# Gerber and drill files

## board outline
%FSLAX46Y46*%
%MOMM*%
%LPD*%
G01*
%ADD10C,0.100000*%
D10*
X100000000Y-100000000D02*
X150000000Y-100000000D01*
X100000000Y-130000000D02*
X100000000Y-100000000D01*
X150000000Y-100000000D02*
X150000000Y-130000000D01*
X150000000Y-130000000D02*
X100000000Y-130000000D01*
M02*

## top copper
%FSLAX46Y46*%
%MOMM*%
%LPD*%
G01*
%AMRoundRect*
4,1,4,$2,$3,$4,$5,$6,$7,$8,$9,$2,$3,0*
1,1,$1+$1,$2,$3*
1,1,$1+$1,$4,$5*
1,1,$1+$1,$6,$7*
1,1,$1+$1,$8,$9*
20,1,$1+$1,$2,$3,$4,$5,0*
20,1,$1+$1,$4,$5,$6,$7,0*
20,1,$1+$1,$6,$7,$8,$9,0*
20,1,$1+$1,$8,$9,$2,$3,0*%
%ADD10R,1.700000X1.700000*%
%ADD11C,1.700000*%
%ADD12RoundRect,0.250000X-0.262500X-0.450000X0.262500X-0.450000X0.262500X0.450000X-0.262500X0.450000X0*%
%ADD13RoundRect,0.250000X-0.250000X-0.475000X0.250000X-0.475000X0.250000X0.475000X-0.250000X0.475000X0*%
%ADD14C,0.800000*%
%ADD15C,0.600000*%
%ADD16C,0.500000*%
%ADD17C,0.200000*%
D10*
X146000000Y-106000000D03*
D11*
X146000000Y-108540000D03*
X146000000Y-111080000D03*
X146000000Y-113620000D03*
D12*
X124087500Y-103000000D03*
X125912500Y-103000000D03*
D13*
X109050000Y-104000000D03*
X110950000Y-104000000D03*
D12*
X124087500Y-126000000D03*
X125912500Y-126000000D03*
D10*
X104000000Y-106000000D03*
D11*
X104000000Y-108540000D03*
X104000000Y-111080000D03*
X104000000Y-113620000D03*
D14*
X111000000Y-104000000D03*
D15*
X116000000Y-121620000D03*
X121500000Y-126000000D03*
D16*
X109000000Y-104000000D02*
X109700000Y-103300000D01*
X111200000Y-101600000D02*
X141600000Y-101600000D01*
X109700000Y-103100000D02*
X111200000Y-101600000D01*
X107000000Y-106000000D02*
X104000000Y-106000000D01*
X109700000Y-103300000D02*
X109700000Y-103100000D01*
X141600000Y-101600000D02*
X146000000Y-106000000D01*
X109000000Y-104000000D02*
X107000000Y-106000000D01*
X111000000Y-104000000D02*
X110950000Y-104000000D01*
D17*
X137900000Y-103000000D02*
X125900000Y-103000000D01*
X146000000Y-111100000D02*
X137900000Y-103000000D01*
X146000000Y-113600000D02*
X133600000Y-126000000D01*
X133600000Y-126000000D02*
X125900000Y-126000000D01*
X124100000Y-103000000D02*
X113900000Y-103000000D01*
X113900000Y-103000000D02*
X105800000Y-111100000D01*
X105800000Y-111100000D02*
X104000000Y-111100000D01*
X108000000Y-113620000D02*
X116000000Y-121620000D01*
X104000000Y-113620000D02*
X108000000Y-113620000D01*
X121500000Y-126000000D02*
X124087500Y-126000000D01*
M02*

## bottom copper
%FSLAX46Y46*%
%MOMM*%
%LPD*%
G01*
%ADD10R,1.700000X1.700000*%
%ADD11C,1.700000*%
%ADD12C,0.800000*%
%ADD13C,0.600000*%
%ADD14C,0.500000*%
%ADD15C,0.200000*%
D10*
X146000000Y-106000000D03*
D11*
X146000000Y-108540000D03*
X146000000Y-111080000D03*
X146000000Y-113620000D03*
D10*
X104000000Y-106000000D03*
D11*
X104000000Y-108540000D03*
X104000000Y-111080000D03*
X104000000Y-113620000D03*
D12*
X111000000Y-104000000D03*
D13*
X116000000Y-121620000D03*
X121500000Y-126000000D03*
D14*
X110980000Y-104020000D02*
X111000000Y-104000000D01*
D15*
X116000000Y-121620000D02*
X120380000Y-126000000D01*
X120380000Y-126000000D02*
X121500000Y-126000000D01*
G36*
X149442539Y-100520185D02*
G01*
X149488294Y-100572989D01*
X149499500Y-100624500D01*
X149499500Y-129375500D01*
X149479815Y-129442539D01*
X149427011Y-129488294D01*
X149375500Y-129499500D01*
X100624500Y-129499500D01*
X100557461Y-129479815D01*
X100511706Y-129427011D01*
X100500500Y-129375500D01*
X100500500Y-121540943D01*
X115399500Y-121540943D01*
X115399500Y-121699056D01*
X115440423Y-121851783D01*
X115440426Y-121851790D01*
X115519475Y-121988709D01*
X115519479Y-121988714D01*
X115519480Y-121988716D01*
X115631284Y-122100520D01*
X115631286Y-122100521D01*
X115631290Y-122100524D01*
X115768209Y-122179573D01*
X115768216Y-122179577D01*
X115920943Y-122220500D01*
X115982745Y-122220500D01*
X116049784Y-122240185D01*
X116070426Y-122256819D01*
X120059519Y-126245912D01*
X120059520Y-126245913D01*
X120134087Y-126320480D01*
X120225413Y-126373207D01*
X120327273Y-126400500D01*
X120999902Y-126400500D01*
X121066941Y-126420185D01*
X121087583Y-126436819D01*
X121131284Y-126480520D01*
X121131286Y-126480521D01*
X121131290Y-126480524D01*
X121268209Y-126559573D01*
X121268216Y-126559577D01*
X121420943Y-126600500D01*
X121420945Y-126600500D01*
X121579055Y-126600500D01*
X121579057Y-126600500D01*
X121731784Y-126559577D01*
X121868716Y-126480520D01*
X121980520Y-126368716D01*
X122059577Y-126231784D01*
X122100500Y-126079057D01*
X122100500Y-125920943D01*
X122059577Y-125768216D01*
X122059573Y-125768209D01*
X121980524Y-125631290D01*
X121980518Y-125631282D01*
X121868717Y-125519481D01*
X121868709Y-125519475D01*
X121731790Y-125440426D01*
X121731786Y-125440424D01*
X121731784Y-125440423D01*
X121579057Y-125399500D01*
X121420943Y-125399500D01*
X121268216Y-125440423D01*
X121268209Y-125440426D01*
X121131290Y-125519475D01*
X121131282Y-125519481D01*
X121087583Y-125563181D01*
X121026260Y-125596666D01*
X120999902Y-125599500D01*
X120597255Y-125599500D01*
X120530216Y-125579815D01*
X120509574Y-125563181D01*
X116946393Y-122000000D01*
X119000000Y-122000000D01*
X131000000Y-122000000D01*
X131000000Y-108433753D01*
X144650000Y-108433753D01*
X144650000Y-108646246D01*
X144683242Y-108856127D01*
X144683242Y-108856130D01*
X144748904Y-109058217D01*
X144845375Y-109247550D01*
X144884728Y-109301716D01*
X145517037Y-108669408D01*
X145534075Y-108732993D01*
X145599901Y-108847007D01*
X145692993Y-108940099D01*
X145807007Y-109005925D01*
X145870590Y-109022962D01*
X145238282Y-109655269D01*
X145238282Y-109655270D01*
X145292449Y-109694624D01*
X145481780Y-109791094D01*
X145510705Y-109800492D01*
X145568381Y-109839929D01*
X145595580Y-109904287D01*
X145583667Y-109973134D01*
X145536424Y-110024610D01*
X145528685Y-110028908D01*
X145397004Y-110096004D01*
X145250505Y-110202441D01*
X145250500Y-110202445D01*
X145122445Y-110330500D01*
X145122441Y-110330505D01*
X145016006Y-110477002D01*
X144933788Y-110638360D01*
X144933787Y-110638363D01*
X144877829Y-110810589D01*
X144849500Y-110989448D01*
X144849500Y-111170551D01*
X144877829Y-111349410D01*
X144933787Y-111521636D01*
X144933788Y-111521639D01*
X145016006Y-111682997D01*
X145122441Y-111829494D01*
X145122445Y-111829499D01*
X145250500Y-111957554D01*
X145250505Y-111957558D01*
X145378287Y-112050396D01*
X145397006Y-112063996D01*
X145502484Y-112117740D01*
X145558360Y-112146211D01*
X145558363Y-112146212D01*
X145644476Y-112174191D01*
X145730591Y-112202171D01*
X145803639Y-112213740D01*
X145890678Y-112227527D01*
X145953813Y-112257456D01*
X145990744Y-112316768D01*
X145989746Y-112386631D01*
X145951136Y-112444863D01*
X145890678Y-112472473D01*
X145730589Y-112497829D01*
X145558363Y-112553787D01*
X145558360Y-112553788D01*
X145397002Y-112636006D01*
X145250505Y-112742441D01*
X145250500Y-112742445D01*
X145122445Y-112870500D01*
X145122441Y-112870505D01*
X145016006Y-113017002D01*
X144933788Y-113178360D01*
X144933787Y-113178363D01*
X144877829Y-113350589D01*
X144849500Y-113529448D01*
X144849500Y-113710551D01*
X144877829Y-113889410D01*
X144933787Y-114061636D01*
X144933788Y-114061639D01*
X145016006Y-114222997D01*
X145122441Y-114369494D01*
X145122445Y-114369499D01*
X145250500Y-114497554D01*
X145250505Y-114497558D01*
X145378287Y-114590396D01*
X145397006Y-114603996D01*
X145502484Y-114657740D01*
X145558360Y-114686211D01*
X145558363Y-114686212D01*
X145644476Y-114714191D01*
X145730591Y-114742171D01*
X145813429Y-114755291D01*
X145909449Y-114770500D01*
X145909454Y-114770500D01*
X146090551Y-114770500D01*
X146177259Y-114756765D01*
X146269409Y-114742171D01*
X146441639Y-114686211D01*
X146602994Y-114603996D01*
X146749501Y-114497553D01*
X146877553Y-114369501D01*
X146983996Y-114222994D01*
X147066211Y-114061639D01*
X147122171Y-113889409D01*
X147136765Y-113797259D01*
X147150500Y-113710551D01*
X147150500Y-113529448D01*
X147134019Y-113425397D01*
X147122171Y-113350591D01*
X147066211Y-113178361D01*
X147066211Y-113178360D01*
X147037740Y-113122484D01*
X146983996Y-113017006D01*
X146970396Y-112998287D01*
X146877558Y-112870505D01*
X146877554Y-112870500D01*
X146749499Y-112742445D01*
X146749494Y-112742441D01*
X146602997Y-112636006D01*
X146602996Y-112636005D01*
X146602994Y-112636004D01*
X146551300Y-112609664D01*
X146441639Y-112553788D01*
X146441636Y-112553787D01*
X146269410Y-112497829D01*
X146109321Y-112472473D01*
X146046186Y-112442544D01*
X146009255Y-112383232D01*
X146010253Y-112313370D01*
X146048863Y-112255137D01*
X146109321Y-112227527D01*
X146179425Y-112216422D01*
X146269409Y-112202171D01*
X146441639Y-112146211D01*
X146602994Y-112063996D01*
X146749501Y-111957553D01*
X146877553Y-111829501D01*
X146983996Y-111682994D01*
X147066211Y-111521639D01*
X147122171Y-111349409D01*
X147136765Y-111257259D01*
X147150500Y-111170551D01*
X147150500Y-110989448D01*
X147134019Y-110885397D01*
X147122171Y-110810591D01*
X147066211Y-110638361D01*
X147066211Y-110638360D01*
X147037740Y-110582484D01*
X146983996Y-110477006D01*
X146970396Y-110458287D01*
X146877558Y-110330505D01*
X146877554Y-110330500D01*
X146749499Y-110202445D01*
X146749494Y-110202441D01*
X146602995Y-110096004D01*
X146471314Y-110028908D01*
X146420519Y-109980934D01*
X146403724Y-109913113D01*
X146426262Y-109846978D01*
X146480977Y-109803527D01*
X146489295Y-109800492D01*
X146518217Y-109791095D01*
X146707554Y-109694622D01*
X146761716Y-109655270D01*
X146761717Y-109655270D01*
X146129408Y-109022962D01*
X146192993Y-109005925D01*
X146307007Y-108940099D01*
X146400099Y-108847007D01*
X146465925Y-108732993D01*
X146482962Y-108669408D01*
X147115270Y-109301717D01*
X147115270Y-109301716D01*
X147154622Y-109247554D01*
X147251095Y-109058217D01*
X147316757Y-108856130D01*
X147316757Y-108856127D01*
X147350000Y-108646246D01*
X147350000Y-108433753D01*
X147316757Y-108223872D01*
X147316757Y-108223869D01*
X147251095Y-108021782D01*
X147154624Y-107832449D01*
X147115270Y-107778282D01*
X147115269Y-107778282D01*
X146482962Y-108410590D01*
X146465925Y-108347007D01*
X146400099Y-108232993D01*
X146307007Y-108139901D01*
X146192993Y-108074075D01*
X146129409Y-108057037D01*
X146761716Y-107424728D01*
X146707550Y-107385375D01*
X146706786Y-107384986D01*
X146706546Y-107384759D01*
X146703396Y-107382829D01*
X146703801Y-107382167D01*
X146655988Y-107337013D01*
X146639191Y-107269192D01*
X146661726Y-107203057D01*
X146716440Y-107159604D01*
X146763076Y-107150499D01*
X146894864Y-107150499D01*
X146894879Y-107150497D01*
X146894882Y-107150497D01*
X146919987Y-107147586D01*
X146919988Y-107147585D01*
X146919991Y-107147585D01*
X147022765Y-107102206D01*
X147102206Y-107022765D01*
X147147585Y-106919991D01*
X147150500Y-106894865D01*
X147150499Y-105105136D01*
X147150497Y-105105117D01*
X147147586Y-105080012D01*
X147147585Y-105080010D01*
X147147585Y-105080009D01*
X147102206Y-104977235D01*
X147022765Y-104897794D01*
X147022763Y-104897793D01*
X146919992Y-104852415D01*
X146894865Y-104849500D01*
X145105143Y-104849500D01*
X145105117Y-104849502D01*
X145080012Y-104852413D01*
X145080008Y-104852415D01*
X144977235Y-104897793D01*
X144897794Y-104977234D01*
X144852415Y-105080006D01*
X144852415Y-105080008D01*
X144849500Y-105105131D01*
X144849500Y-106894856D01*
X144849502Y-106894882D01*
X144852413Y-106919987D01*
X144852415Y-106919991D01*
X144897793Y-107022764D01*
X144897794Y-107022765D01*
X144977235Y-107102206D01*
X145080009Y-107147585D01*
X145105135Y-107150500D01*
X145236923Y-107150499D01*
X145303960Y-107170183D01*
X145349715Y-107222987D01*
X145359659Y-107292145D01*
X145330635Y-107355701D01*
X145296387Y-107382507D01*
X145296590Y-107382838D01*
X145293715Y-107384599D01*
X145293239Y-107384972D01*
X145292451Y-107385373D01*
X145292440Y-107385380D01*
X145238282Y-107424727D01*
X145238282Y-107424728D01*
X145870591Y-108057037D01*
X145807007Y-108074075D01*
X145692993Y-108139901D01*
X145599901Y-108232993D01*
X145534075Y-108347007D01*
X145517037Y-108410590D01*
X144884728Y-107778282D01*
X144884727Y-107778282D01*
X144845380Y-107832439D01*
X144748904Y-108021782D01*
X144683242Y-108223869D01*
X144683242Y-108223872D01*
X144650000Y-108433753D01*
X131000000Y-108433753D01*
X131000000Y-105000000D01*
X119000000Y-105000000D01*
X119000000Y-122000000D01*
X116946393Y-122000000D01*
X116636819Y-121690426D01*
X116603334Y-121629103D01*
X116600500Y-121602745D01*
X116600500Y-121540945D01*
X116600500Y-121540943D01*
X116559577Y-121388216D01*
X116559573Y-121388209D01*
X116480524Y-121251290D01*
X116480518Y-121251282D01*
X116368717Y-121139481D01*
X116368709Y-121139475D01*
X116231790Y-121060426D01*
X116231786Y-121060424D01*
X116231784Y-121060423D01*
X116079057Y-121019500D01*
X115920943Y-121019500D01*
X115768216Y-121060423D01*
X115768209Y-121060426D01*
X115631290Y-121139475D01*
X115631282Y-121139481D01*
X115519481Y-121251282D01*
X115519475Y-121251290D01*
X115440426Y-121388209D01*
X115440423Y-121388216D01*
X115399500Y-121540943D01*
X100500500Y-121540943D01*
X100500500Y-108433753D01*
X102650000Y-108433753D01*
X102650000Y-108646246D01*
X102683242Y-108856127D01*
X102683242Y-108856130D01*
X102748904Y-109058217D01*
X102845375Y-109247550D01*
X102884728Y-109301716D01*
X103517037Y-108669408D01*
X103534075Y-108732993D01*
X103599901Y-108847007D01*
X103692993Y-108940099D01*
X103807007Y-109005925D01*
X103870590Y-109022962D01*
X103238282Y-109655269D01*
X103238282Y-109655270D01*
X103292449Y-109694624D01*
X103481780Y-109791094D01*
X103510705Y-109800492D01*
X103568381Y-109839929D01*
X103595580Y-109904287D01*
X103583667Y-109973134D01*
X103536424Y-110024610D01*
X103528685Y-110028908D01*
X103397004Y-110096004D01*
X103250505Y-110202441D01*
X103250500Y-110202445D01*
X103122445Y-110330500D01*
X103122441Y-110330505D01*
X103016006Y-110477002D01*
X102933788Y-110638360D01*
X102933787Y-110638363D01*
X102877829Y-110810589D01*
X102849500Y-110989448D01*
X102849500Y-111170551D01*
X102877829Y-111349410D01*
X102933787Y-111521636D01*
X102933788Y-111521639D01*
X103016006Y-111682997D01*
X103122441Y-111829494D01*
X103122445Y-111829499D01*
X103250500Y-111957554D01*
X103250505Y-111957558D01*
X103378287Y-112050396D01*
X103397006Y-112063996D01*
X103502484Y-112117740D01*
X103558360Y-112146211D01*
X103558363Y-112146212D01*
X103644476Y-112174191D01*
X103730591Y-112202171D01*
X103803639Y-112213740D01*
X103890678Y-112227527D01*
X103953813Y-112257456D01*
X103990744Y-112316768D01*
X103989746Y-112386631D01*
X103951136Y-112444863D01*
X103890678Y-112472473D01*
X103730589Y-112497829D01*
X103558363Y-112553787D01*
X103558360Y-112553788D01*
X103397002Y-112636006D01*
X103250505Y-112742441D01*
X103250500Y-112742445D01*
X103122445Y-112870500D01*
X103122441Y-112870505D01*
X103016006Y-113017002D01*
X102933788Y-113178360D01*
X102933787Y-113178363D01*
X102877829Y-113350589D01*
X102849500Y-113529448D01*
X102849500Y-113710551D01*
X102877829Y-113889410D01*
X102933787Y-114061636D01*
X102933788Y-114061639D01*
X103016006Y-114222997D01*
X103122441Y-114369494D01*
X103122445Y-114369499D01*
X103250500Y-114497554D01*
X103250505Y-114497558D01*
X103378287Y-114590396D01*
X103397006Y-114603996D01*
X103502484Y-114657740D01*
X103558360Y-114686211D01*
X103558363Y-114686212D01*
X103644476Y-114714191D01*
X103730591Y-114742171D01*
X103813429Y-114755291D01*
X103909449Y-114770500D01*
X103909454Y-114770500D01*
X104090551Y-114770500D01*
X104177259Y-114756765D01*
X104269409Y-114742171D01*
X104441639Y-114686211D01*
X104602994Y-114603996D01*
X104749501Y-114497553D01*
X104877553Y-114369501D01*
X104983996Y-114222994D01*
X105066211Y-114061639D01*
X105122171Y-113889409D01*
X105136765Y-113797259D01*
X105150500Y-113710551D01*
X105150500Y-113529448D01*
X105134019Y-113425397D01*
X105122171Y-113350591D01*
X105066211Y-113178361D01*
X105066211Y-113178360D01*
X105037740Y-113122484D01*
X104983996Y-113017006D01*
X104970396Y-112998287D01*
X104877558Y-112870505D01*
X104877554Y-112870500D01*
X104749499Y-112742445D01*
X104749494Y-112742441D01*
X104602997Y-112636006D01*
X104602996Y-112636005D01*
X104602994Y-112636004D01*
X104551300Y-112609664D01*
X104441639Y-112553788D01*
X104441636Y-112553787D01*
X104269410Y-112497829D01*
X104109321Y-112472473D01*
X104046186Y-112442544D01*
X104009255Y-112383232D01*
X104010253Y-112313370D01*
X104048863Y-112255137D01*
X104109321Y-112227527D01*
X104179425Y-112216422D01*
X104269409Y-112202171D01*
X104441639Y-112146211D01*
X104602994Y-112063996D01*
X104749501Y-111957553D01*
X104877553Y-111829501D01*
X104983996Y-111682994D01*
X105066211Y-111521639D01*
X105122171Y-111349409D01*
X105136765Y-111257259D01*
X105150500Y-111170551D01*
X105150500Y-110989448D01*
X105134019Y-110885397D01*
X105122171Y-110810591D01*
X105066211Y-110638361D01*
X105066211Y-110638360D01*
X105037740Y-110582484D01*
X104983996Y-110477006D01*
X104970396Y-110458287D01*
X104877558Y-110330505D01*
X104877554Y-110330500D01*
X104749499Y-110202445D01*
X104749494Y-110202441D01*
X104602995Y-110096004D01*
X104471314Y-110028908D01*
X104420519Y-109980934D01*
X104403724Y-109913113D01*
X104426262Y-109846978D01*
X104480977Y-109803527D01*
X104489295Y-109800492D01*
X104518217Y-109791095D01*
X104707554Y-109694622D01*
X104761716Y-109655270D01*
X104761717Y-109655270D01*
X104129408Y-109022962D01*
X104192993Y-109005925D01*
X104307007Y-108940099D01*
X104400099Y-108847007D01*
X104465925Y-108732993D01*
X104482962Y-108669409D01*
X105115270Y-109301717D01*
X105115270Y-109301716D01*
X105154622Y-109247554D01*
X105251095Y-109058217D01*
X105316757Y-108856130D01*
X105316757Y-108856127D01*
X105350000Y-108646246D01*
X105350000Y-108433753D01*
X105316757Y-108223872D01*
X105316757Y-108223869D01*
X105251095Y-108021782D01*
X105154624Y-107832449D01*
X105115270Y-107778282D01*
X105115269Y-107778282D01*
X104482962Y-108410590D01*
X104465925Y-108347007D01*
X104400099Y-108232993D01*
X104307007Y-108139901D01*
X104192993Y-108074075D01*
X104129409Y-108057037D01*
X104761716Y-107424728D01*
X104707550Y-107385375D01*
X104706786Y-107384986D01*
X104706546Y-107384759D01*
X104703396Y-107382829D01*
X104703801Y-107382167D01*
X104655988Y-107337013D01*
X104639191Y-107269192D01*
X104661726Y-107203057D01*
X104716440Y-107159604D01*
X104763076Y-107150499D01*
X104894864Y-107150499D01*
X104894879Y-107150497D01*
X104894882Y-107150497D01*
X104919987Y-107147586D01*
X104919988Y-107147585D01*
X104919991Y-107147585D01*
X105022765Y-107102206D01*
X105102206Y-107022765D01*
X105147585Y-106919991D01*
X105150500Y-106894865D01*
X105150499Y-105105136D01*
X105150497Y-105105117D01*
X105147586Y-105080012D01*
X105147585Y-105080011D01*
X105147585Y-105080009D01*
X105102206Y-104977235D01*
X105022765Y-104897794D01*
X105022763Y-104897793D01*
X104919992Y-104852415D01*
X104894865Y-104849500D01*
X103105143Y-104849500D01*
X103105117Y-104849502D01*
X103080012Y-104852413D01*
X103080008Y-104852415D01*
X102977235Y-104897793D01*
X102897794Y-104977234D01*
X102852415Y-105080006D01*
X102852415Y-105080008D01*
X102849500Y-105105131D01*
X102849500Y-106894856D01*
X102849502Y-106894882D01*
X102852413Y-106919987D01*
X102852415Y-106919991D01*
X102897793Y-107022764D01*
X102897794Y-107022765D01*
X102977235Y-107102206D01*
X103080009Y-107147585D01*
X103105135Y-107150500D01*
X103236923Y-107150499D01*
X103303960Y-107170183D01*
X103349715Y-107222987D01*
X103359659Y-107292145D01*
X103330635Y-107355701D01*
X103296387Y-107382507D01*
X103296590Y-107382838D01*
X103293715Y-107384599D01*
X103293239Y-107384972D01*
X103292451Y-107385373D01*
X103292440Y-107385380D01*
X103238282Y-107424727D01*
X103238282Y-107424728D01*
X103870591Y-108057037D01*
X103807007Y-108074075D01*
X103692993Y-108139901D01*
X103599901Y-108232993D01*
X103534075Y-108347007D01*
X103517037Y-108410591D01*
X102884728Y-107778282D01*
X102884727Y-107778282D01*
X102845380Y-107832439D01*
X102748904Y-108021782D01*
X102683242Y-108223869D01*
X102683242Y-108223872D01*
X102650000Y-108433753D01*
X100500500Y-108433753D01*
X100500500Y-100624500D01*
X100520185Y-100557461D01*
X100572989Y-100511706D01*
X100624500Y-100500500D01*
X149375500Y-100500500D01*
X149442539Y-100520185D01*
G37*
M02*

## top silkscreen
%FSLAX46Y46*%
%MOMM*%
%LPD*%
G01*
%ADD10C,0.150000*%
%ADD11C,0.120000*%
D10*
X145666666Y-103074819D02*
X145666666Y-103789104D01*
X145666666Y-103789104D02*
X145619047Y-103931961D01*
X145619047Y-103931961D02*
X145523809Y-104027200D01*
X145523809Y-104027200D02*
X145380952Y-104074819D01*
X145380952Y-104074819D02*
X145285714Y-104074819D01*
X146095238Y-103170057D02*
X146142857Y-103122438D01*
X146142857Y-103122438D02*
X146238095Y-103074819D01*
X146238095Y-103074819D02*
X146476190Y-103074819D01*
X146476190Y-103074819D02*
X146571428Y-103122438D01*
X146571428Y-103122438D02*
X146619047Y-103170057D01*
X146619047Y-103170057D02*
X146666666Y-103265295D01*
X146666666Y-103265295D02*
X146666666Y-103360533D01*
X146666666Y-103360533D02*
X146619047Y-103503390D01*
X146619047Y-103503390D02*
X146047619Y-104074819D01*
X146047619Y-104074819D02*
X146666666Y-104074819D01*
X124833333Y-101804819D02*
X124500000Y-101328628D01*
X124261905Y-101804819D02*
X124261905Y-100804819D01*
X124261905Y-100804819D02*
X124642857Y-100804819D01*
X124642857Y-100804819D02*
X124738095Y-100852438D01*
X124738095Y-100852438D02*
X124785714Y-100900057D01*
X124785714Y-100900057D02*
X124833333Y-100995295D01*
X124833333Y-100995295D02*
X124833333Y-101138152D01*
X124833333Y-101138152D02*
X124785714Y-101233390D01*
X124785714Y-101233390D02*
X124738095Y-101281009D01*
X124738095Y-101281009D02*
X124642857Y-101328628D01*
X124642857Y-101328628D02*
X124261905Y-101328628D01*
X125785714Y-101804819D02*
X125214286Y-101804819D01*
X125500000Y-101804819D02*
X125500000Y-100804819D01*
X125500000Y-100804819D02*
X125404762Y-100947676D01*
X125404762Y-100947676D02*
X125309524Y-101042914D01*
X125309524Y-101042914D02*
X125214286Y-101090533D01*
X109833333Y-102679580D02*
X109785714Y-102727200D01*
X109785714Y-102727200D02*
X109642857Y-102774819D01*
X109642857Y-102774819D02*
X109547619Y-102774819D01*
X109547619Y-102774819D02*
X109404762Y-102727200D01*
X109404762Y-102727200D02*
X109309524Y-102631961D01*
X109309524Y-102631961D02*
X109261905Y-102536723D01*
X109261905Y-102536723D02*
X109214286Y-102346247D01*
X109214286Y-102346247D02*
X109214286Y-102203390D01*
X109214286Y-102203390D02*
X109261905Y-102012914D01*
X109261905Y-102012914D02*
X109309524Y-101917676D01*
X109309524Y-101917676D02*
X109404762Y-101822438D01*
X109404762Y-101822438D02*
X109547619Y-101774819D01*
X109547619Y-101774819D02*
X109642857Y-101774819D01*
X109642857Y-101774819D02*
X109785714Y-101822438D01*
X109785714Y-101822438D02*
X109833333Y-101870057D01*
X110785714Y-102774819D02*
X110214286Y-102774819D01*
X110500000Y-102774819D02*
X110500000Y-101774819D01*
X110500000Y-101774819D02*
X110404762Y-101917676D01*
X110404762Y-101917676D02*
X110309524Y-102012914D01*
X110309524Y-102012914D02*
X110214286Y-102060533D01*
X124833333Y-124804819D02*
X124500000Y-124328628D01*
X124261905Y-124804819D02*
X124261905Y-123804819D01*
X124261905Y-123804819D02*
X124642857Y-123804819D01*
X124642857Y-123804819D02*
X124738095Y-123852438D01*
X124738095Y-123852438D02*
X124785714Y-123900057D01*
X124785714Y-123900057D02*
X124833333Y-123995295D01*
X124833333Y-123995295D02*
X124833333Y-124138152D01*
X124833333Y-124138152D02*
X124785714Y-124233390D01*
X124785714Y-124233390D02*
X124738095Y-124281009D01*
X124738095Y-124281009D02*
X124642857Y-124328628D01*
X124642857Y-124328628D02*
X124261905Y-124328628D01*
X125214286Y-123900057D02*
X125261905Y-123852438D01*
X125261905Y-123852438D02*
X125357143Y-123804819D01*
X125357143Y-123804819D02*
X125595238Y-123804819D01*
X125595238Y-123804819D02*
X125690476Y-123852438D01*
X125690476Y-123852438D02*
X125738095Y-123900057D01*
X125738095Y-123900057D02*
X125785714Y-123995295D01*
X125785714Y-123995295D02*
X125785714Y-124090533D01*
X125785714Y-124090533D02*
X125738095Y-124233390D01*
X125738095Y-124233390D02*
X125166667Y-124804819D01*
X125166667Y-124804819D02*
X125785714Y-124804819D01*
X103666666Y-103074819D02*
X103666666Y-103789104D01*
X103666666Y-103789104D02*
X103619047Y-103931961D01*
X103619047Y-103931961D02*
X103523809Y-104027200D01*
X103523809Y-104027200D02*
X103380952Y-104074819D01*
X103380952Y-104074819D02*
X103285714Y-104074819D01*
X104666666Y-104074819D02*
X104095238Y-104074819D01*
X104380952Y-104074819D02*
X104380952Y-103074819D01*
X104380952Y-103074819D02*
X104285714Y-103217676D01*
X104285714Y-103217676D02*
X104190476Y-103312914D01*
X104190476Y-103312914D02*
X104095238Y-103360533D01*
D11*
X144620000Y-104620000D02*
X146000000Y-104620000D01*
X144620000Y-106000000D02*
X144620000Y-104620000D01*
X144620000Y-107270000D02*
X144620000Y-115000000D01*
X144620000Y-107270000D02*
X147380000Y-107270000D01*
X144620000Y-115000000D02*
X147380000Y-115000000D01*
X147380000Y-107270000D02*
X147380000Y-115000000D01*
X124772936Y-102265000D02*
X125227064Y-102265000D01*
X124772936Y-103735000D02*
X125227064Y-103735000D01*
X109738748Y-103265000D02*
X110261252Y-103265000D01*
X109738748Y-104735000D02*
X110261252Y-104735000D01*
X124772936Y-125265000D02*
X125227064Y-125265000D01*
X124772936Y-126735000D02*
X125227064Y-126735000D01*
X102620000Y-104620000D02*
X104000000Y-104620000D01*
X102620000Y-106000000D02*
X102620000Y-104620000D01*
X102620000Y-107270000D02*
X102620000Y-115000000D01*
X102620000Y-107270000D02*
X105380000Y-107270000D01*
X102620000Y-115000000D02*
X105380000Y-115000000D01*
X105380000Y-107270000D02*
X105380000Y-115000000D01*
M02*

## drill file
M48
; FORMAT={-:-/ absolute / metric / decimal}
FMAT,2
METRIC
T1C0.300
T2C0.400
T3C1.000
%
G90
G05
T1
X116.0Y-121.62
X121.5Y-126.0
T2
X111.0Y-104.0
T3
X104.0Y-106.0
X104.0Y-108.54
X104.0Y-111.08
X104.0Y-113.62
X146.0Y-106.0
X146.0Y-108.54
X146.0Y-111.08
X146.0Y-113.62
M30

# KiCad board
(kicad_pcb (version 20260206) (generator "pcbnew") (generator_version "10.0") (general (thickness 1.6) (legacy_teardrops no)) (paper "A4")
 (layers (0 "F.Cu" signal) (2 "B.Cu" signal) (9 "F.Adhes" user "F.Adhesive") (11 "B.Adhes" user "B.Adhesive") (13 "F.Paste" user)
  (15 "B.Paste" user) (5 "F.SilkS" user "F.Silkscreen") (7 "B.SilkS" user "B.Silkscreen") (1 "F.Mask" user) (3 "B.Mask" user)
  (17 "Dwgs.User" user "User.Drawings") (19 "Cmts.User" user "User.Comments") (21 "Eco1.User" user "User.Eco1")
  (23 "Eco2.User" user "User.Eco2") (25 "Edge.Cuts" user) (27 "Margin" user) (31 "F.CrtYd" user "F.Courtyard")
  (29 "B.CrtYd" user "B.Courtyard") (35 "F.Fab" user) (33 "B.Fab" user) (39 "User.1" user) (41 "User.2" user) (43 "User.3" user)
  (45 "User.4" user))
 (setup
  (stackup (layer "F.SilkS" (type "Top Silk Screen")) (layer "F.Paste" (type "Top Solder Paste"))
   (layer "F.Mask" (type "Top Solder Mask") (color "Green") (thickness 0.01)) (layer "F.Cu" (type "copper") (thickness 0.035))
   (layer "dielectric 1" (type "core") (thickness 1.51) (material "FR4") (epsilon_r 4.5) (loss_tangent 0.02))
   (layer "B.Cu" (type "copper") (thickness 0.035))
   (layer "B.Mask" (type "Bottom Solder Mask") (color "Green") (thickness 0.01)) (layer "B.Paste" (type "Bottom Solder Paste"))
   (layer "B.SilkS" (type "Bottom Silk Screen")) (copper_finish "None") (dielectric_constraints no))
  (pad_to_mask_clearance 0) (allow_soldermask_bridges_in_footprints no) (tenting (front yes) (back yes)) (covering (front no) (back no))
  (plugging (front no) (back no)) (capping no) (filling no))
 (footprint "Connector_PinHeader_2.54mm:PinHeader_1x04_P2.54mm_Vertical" (layer "F.Cu") (at 146 106)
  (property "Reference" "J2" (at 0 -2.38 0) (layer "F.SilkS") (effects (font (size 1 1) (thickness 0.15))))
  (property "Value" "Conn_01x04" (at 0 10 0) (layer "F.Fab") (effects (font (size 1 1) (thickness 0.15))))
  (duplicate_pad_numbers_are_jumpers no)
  (fp_line (start -1.38 -1.38) (end 0 -1.38) (stroke (width 0.12) (type solid)) (layer "F.SilkS"))
  (fp_line (start -1.38 0) (end -1.38 -1.38) (stroke (width 0.12) (type solid)) (layer "F.SilkS"))
  (fp_line (start -1.38 1.27) (end -1.38 9) (stroke (width 0.12) (type solid)) (layer "F.SilkS"))
  (fp_line (start -1.38 1.27) (end 1.38 1.27) (stroke (width 0.12) (type solid)) (layer "F.SilkS"))
  (fp_line (start -1.38 9) (end 1.38 9) (stroke (width 0.12) (type solid)) (layer "F.SilkS"))
  (fp_line (start 1.38 1.27) (end 1.38 9) (stroke (width 0.12) (type solid)) (layer "F.SilkS"))
  (pad "1" thru_hole rect (at 0 0) (size 1.7 1.7) (drill 1) (layers "*.Cu" "*.Mask") (remove_unused_layers no) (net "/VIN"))
  (pad "2" thru_hole circle (at 0 2.54) (size 1.7 1.7) (drill 1) (layers "*.Cu" "*.Mask") (remove_unused_layers no) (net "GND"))
  (pad "3" thru_hole circle (at 0 5.08) (size 1.7 1.7) (drill 1) (layers "*.Cu" "*.Mask") (remove_unused_layers no) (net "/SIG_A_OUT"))
  (pad "4" thru_hole circle (at 0 7.62) (size 1.7 1.7) (drill 1) (layers "*.Cu" "*.Mask") (remove_unused_layers no) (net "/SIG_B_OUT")))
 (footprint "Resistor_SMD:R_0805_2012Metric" (layer "F.Cu") (at 125 103)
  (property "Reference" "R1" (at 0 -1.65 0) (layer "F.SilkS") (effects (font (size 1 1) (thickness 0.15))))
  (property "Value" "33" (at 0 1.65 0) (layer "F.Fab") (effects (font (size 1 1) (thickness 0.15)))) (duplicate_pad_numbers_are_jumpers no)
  (fp_line (start -0.227064 -0.735) (end 0.227064 -0.735) (stroke (width 0.12) (type solid)) (layer "F.SilkS"))
  (fp_line (start -0.227064 0.735) (end 0.227064 0.735) (stroke (width 0.12) (type solid)) (layer "F.SilkS"))
  (pad "1" smd roundrect (at -0.9125 0) (size 1.025 1.4) (layers "F.Cu" "F.Mask" "F.Paste") (roundrect_rratio 0.243902) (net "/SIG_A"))
  (pad "2" smd roundrect (at 0.9125 0) (size 1.025 1.4) (layers "F.Cu" "F.Mask" "F.Paste") (roundrect_rratio 0.243902) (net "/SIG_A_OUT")))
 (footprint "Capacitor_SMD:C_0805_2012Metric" (layer "F.Cu") (at 110 104)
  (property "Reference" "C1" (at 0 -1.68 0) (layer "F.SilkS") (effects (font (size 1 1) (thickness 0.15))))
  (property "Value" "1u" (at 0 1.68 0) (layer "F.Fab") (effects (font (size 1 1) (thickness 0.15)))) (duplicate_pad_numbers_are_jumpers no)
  (fp_line (start -0.261252 -0.735) (end 0.261252 -0.735) (stroke (width 0.12) (type solid)) (layer "F.SilkS"))
  (fp_line (start -0.261252 0.735) (end 0.261252 0.735) (stroke (width 0.12) (type solid)) (layer "F.SilkS"))
  (pad "1" smd roundrect (at -0.95 0) (size 1 1.45) (layers "F.Cu" "F.Mask" "F.Paste") (roundrect_rratio 0.25) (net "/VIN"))
  (pad "2" smd roundrect (at 0.95 0) (size 1 1.45) (layers "F.Cu" "F.Mask" "F.Paste") (roundrect_rratio 0.25) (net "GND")))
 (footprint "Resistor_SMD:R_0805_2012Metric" (layer "F.Cu") (at 125 126)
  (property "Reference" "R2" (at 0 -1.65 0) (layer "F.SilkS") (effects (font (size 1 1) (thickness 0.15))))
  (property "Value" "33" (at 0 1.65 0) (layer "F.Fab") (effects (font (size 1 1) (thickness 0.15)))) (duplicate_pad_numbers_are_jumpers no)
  (fp_line (start -0.227064 -0.735) (end 0.227064 -0.735) (stroke (width 0.12) (type solid)) (layer "F.SilkS"))
  (fp_line (start -0.227064 0.735) (end 0.227064 0.735) (stroke (width 0.12) (type solid)) (layer "F.SilkS"))
  (pad "1" smd roundrect (at -0.9125 0) (size 1.025 1.4) (layers "F.Cu" "F.Mask" "F.Paste") (roundrect_rratio 0.243902) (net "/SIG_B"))
  (pad "2" smd roundrect (at 0.9125 0) (size 1.025 1.4) (layers "F.Cu" "F.Mask" "F.Paste") (roundrect_rratio 0.243902) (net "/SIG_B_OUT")))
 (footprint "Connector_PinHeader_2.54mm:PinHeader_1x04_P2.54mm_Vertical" (layer "F.Cu") (at 104 106)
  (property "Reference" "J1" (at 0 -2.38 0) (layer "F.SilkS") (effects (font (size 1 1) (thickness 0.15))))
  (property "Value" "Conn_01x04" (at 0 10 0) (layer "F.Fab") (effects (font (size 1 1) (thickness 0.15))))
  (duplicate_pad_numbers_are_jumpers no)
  (fp_line (start -1.38 -1.38) (end 0 -1.38) (stroke (width 0.12) (type solid)) (layer "F.SilkS"))
  (fp_line (start -1.38 0) (end -1.38 -1.38) (stroke (width 0.12) (type solid)) (layer "F.SilkS"))
  (fp_line (start -1.38 1.27) (end -1.38 9) (stroke (width 0.12) (type solid)) (layer "F.SilkS"))
  (fp_line (start -1.38 1.27) (end 1.38 1.27) (stroke (width 0.12) (type solid)) (layer "F.SilkS"))
  (fp_line (start -1.38 9) (end 1.38 9) (stroke (width 0.12) (type solid)) (layer "F.SilkS"))
  (fp_line (start 1.38 1.27) (end 1.38 9) (stroke (width 0.12) (type solid)) (layer "F.SilkS"))
  (pad "1" thru_hole rect (at 0 0) (size 1.7 1.7) (drill 1) (layers "*.Cu" "*.Mask") (remove_unused_layers no) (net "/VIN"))
  (pad "2" thru_hole circle (at 0 2.54) (size 1.7 1.7) (drill 1) (layers "*.Cu" "*.Mask") (remove_unused_layers no) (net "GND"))
  (pad "3" thru_hole circle (at 0 5.08) (size 1.7 1.7) (drill 1) (layers "*.Cu" "*.Mask") (remove_unused_layers no) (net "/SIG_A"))
  (pad "4" thru_hole circle (at 0 7.62) (size 1.7 1.7) (drill 1) (layers "*.Cu" "*.Mask") (remove_unused_layers no) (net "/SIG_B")))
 (gr_line (start 100 100) (end 150 100) (stroke (width 0.1) (type default)) (layer "Edge.Cuts"))
 (gr_line (start 100 130) (end 100 100) (stroke (width 0.1) (type default)) (layer "Edge.Cuts"))
 (gr_line (start 150 100) (end 150 130) (stroke (width 0.1) (type default)) (layer "Edge.Cuts"))
 (gr_line (start 150 130) (end 100 130) (stroke (width 0.1) (type default)) (layer "Edge.Cuts"))
 (segment (start 109 104) (end 109.7 103.3) (width 0.5) (layer "F.Cu") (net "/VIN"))
 (segment (start 111.2 101.6) (end 141.6 101.6) (width 0.5) (layer "F.Cu") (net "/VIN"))
 (segment (start 109.7 103.1) (end 111.2 101.6) (width 0.5) (layer "F.Cu") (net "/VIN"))
 (segment (start 107 106) (end 104 106) (width 0.5) (layer "F.Cu") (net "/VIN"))
 (segment (start 109.7 103.3) (end 109.7 103.1) (width 0.5) (layer "F.Cu") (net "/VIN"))
 (segment (start 141.6 101.6) (end 146 106) (width 0.5) (layer "F.Cu") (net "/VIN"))
 (segment (start 109 104) (end 107 106) (width 0.5) (layer "F.Cu") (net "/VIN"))
 (segment (start 111 104) (end 110.95 104) (width 0.5) (layer "F.Cu") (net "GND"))
 (via (at 111 104) (size 0.8) (drill 0.4) (layers "F.Cu" "B.Cu") (capping yes) (filling yes) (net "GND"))
 (segment (start 110.98 104.02) (end 111 104) (width 0.5) (layer "B.Cu") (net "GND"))
 (segment (start 137.9 103) (end 125.9 103) (width 0.2) (layer "F.Cu") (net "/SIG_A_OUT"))
 (segment (start 146 111.1) (end 137.9 103) (width 0.2) (layer "F.Cu") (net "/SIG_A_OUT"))
 (segment (start 146 113.6) (end 133.6 126) (width 0.2) (layer "F.Cu") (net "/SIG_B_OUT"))
 (segment (start 133.6 126) (end 125.9 126) (width 0.2) (layer "F.Cu") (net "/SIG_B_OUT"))
 (segment (start 124.1 103) (end 113.9 103) (width 0.2) (layer "F.Cu") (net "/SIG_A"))
 (segment (start 113.9 103) (end 105.8 111.1) (width 0.2) (layer "F.Cu") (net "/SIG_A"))
 (segment (start 105.8 111.1) (end 104 111.1) (width 0.2) (layer "F.Cu") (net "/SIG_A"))
 (segment (start 108 113.62) (end 116 121.62) (width 0.2) (locked yes) (layer "F.Cu") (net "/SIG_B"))
 (segment (start 104 113.62) (end 108 113.62) (width 0.2) (locked yes) (layer "F.Cu") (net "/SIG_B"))
 (segment (start 121.5 126) (end 124.0875 126) (width 0.2) (locked yes) (layer "F.Cu") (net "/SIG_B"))
 (via (at 116 121.62) (size 0.6) (drill 0.3) (layers "F.Cu" "B.Cu") (locked yes) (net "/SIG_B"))
 (via (at 121.5 126) (size 0.6) (drill 0.3) (layers "F.Cu" "B.Cu") (locked yes) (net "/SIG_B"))
 (segment (start 116 121.62) (end 120.38 126) (width 0.2) (locked yes) (layer "B.Cu") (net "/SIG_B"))
 (segment (start 120.38 126) (end 121.5 126) (width 0.2) (locked yes) (layer "B.Cu") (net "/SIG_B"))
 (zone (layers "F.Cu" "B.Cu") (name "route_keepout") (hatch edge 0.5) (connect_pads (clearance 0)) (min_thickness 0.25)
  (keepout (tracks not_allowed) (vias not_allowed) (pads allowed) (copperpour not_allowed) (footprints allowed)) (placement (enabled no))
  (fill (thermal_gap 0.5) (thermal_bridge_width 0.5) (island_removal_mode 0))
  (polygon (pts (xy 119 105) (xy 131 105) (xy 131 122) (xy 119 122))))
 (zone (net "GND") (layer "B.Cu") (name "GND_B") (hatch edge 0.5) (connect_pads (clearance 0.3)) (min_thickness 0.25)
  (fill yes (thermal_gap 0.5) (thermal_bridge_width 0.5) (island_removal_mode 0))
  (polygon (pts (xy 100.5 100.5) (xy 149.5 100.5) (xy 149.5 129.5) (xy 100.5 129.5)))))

